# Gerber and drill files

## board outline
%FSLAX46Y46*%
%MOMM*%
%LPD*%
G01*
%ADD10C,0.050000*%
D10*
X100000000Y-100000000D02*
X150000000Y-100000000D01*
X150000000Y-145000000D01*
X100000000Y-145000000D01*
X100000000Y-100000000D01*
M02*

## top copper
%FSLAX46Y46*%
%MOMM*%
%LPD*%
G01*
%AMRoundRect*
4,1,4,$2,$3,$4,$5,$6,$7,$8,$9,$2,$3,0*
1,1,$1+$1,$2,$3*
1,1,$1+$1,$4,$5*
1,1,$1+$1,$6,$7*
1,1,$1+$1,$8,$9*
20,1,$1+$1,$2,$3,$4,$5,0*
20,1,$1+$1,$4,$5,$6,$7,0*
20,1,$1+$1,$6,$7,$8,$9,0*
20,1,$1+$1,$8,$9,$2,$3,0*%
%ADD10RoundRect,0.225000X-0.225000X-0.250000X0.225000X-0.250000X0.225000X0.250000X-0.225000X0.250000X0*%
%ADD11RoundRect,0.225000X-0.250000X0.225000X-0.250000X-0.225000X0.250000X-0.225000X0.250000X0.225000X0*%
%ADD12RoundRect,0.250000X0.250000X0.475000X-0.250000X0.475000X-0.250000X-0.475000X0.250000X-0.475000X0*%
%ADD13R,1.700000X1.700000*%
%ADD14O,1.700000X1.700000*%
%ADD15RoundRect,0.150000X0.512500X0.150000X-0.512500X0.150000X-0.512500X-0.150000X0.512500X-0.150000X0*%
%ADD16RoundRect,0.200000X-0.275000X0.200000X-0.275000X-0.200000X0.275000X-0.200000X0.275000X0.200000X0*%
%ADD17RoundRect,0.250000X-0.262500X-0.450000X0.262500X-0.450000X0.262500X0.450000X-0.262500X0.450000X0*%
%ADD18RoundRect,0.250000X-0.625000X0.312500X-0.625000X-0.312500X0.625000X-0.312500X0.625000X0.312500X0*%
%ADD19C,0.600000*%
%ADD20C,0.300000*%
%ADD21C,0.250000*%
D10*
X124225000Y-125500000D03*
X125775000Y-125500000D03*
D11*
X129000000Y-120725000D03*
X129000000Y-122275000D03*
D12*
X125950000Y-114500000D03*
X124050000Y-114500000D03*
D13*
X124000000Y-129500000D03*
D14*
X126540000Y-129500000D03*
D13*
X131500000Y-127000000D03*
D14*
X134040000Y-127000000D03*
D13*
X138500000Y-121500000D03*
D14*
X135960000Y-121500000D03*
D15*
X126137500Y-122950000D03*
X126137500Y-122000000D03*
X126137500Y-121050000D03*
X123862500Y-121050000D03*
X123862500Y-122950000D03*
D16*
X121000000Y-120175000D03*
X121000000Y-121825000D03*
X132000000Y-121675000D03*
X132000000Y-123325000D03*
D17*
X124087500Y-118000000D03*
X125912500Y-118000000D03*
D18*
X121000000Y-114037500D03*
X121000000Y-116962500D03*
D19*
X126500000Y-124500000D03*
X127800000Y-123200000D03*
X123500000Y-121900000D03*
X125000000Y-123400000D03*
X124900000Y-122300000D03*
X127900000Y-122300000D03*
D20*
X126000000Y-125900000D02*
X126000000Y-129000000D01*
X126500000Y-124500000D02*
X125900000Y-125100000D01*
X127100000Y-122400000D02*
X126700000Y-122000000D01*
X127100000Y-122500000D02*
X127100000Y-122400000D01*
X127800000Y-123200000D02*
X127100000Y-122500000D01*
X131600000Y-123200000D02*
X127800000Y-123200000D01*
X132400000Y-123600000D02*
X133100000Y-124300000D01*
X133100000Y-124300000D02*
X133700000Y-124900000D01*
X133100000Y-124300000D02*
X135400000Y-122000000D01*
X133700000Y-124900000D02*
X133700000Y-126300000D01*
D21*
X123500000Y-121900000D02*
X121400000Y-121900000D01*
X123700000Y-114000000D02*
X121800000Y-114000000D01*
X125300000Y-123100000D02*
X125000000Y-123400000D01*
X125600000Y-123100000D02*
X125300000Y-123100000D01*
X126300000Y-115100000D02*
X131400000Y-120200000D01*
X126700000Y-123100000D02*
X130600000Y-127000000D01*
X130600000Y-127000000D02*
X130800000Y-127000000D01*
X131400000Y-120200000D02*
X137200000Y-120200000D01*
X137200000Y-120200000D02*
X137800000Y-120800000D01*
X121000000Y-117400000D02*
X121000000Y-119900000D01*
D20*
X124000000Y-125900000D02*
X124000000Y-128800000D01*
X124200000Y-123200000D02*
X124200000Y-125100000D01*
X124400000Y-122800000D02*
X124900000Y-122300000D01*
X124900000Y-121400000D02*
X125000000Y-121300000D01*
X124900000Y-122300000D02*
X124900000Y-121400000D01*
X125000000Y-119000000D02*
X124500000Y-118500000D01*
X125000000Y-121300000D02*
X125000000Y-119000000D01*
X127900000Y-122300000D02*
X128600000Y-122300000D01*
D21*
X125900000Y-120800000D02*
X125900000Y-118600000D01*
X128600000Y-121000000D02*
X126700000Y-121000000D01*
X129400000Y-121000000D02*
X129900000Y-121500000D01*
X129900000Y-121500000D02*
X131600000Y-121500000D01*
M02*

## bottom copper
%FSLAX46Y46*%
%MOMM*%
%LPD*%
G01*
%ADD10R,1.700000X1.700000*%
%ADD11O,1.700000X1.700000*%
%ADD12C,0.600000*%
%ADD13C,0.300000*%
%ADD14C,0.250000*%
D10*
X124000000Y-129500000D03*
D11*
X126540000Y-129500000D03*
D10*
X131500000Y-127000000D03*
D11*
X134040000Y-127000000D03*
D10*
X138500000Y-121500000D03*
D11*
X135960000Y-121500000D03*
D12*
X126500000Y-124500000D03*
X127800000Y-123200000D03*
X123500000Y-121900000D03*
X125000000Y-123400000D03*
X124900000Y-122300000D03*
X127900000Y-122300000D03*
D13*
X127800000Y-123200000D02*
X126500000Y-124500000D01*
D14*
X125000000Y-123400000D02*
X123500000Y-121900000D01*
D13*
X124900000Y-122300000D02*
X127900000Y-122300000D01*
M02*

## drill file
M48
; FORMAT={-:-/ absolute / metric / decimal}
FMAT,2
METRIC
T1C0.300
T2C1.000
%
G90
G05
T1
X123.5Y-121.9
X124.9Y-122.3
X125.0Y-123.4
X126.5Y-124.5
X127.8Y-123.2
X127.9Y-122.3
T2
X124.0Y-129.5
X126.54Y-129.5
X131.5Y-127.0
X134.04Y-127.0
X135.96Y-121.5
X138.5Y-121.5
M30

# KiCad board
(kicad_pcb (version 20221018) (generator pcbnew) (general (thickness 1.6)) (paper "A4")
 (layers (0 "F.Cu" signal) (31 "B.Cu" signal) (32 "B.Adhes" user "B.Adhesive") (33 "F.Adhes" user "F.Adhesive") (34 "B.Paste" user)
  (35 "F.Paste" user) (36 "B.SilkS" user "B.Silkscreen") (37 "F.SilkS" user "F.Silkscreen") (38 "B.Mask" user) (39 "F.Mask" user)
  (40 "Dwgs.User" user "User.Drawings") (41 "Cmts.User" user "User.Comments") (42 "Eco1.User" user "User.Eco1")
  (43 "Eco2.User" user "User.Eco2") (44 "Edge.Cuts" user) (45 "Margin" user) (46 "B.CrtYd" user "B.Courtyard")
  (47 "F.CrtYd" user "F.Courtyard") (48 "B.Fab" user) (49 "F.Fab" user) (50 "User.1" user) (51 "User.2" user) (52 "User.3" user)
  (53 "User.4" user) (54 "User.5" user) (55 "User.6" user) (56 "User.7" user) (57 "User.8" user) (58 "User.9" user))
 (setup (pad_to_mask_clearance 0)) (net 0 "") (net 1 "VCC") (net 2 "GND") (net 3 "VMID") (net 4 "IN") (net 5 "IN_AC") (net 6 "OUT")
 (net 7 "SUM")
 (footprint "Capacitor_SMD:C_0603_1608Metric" (layer "F.Cu") (at 125 125.5)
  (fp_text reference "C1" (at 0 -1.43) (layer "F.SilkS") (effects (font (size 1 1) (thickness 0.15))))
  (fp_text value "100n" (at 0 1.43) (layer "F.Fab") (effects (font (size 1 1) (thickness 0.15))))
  (pad "1" smd roundrect (at -0.775 0) (size 0.9 0.95) (layers "F.Cu" "F.Paste" "F.Mask") (roundrect_rratio 0.25) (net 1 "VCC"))
  (pad "2" smd roundrect (at 0.775 0) (size 0.9 0.95) (layers "F.Cu" "F.Paste" "F.Mask") (roundrect_rratio 0.25) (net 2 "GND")))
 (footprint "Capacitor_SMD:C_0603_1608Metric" (layer "F.Cu") (at 129 121.5 -90)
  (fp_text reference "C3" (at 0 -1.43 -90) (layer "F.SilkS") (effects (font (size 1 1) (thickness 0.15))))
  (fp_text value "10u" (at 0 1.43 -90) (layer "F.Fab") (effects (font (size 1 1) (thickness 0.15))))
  (pad "1" smd roundrect (at -0.775 0 270) (size 0.9 0.95) (layers "F.Cu" "F.Paste" "F.Mask") (roundrect_rratio 0.25) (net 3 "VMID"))
  (pad "2" smd roundrect (at 0.775 0 270) (size 0.9 0.95) (layers "F.Cu" "F.Paste" "F.Mask") (roundrect_rratio 0.25) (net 1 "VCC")))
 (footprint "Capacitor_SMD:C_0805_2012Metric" (layer "F.Cu") (at 125 114.5 180)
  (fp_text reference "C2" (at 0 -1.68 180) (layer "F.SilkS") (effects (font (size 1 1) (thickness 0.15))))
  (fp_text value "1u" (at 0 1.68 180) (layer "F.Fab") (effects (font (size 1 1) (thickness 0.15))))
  (pad "1" smd roundrect (at -0.95 0 180) (size 1 1.45) (layers "F.Cu" "F.Paste" "F.Mask") (roundrect_rratio 0.25) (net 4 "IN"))
  (pad "2" smd roundrect (at 0.95 0 180) (size 1 1.45) (layers "F.Cu" "F.Paste" "F.Mask") (roundrect_rratio 0.25) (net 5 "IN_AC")))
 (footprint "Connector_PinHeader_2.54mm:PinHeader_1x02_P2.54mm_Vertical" (layer "F.Cu") (at 124 129.5 90)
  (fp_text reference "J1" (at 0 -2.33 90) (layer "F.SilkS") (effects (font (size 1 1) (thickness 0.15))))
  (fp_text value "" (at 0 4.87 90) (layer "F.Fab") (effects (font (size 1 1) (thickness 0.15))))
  (pad "1" thru_hole rect (at 0 0 90) (size 1.7 1.7) (drill 1) (layers "*.Cu" "*.Mask") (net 1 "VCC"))
  (pad "2" thru_hole oval (at 0 2.54 90) (size 1.7 1.7) (drill 1) (layers "*.Cu" "*.Mask") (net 2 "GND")))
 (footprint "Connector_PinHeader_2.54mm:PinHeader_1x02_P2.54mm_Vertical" (layer "F.Cu") (at 131.5 127 90)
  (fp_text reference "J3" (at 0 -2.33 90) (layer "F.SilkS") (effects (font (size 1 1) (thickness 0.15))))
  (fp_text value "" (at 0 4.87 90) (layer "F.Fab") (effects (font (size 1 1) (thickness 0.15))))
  (pad "1" thru_hole rect (at 0 0 90) (size 1.7 1.7) (drill 1) (layers "*.Cu" "*.Mask") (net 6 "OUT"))
  (pad "2" thru_hole oval (at 0 2.54 90) (size 1.7 1.7) (drill 1) (layers "*.Cu" "*.Mask") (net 2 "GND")))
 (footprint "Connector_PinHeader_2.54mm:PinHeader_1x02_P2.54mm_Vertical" (layer "F.Cu") (at 138.5 121.5 -90)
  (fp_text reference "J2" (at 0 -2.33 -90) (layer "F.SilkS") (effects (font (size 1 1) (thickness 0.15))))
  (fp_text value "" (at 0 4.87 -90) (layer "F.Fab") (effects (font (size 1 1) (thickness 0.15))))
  (pad "1" thru_hole rect (at 0 0 270) (size 1.7 1.7) (drill 1) (layers "*.Cu" "*.Mask") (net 4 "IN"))
  (pad "2" thru_hole oval (at 0 2.54 270) (size 1.7 1.7) (drill 1) (layers "*.Cu" "*.Mask") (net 2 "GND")))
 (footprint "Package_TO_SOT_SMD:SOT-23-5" (layer "F.Cu") (at 125 122 180)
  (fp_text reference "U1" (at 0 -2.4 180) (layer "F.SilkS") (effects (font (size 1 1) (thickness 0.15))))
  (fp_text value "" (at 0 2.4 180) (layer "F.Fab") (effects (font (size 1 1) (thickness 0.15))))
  (pad "1" smd roundrect (at -1.1375 -0.95 180) (size 1.325 0.6) (layers "F.Cu" "F.Paste" "F.Mask") (roundrect_rratio 0.25) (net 6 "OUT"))
  (pad "2" smd roundrect (at -1.1375 0 180) (size 1.325 0.6) (layers "F.Cu" "F.Paste" "F.Mask") (roundrect_rratio 0.25) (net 2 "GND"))
  (pad "3" smd roundrect (at -1.1375 0.95 180) (size 1.325 0.6) (layers "F.Cu" "F.Paste" "F.Mask") (roundrect_rratio 0.25) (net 3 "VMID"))
  (pad "4" smd roundrect (at 1.1375 0.95 180) (size 1.325 0.6) (layers "F.Cu" "F.Paste" "F.Mask") (roundrect_rratio 0.25))
  (pad "5" smd roundrect (at 1.1375 -0.95 180) (size 1.325 0.6) (layers "F.Cu" "F.Paste" "F.Mask") (roundrect_rratio 0.25) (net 1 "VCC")))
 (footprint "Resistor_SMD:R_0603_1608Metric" (layer "F.Cu") (at 121 121 -90)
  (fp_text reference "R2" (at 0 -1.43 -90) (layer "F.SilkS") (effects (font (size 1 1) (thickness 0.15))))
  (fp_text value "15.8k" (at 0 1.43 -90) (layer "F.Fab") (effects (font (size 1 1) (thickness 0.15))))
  (pad "1" smd roundrect (at -0.825 0 270) (size 0.8 0.95) (layers "F.Cu" "F.Paste" "F.Mask") (roundrect_rratio 0.25) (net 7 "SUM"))
  (pad "2" smd roundrect (at 0.825 0 270) (size 0.8 0.95) (layers "F.Cu" "F.Paste" "F.Mask") (roundrect_rratio 0.25) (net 6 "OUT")))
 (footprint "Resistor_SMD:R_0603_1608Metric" (layer "F.Cu") (at 132 122.5 -90)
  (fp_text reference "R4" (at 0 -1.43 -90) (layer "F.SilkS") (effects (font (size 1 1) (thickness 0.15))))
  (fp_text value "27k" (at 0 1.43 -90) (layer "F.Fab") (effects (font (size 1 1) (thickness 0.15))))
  (pad "1" smd roundrect (at -0.825 0 270) (size 0.8 0.95) (layers "F.Cu" "F.Paste" "F.Mask") (roundrect_rratio 0.25) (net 3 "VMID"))
  (pad "2" smd roundrect (at 0.825 0 270) (size 0.8 0.95) (layers "F.Cu" "F.Paste" "F.Mask") (roundrect_rratio 0.25) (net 2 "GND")))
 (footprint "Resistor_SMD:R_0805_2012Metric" (layer "F.Cu") (at 125 118)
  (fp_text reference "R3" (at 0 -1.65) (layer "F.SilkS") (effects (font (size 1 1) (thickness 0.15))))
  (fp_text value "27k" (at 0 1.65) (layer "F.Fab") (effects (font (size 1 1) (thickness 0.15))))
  (pad "1" smd roundrect (at -0.9125 0) (size 1.025 1.4) (layers "F.Cu" "F.Paste" "F.Mask") (roundrect_rratio 0.243902) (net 1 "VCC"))
  (pad "2" smd roundrect (at 0.9125 0) (size 1.025 1.4) (layers "F.Cu" "F.Paste" "F.Mask") (roundrect_rratio 0.243902) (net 3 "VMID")))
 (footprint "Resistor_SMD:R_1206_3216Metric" (layer "F.Cu") (at 121 115.5 -90)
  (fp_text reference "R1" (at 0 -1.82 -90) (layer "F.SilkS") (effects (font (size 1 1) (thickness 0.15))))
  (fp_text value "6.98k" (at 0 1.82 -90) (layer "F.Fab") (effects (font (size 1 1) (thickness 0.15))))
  (pad "1" smd roundrect (at -1.4625 0 270) (size 1.125 1.75) (layers "F.Cu" "F.Paste" "F.Mask") (roundrect_rratio 0.222222) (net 5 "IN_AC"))
  (pad "2" smd roundrect (at 1.4625 0 270) (size 1.125 1.75) (layers "F.Cu" "F.Paste" "F.Mask") (roundrect_rratio 0.222222) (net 7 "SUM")))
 (gr_rect (start 100 100) (end 150 145) (stroke (width 0.05) (type default)) (fill none) (layer "Edge.Cuts"))
 (segment (start 126 125.9) (end 126 129) (width 0.3) (layer "F.Cu") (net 2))
 (segment (start 126.5 124.5) (end 125.9 125.1) (width 0.3) (layer "F.Cu") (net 2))
 (segment (start 127.1 122.4) (end 126.7 122) (width 0.3) (layer "F.Cu") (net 2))
 (segment (start 127.1 122.5) (end 127.1 122.4) (width 0.3) (layer "F.Cu") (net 2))
 (segment (start 127.8 123.2) (end 127.1 122.5) (width 0.3) (layer "F.Cu") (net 2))
 (segment (start 131.6 123.2) (end 127.8 123.2) (width 0.3) (layer "F.Cu") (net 2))
 (segment (start 132.4 123.6) (end 133.1 124.3) (width 0.3) (layer "F.Cu") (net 2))
 (segment (start 133.1 124.3) (end 133.7 124.9) (width 0.3) (layer "F.Cu") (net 2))
 (segment (start 133.1 124.3) (end 135.4 122) (width 0.3) (layer "F.Cu") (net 2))
 (segment (start 133.7 124.9) (end 133.7 126.3) (width 0.3) (layer "F.Cu") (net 2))
 (via (at 126.5 124.5) (size 0.6) (drill 0.3) (layers "F.Cu" "B.Cu") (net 2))
 (via (at 127.8 123.2) (size 0.6) (drill 0.3) (layers "F.Cu" "B.Cu") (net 2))
 (segment (start 123.5 121.9) (end 121.4 121.9) (width 0.25) (layer "F.Cu") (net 6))
 (segment (start 123.7 114) (end 121.8 114) (width 0.25) (layer "F.Cu") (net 5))
 (segment (start 125.3 123.1) (end 125 123.4) (width 0.25) (layer "F.Cu") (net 6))
 (segment (start 125.6 123.1) (end 125.3 123.1) (width 0.25) (layer "F.Cu") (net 6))
 (segment (start 126.3 115.1) (end 131.4 120.2) (width 0.25) (layer "F.Cu") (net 4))
 (segment (start 126.7 123.1) (end 130.6 127) (width 0.25) (layer "F.Cu") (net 6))
 (segment (start 127.8 123.2) (end 126.5 124.5) (width 0.3) (layer "B.Cu") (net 2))
 (segment (start 130.6 127) (end 130.8 127) (width 0.25) (layer "F.Cu") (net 6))
 (segment (start 131.4 120.2) (end 137.2 120.2) (width 0.25) (layer "F.Cu") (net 4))
 (segment (start 137.2 120.2) (end 137.8 120.8) (width 0.25) (layer "F.Cu") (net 4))
 (via (at 123.5 121.9) (size 0.6) (drill 0.3) (layers "F.Cu" "B.Cu") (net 6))
 (via (at 125 123.4) (size 0.6) (drill 0.3) (layers "F.Cu" "B.Cu") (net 6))
 (segment (start 121 117.4) (end 121 119.9) (width 0.25) (layer "F.Cu") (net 7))
 (segment (start 124 125.9) (end 124 128.8) (width 0.3) (layer "F.Cu") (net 1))
 (segment (start 124.2 123.2) (end 124.2 125.1) (width 0.3) (layer "F.Cu") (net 1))
 (segment (start 124.4 122.8) (end 124.9 122.3) (width 0.3) (layer "F.Cu") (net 1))
 (segment (start 124.9 121.4) (end 125 121.3) (width 0.3) (layer "F.Cu") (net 1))
 (segment (start 124.9 122.3) (end 124.9 121.4) (width 0.3) (layer "F.Cu") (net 1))
 (segment (start 125 119) (end 124.5 118.5) (width 0.3) (layer "F.Cu") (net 1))
 (segment (start 125 121.3) (end 125 119) (width 0.3) (layer "F.Cu") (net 1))
 (segment (start 125 123.4) (end 123.5 121.9) (width 0.25) (layer "B.Cu") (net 6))
 (segment (start 127.9 122.3) (end 128.6 122.3) (width 0.3) (layer "F.Cu") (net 1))
 (via (at 124.9 122.3) (size 0.6) (drill 0.3) (layers "F.Cu" "B.Cu") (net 1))
 (via (at 127.9 122.3) (size 0.6) (drill 0.3) (layers "F.Cu" "B.Cu") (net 1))
 (segment (start 124.9 122.3) (end 127.9 122.3) (width 0.3) (layer "B.Cu") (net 1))
 (segment (start 125.9 120.8) (end 125.9 118.6) (width 0.25) (layer "F.Cu") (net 3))
 (segment (start 128.6 121) (end 126.7 121) (width 0.25) (layer "F.Cu") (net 3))
 (segment (start 129.4 121) (end 129.9 121.5) (width 0.25) (layer "F.Cu") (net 3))
 (segment (start 129.9 121.5) (end 131.6 121.5) (width 0.25) (layer "F.Cu") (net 3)))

